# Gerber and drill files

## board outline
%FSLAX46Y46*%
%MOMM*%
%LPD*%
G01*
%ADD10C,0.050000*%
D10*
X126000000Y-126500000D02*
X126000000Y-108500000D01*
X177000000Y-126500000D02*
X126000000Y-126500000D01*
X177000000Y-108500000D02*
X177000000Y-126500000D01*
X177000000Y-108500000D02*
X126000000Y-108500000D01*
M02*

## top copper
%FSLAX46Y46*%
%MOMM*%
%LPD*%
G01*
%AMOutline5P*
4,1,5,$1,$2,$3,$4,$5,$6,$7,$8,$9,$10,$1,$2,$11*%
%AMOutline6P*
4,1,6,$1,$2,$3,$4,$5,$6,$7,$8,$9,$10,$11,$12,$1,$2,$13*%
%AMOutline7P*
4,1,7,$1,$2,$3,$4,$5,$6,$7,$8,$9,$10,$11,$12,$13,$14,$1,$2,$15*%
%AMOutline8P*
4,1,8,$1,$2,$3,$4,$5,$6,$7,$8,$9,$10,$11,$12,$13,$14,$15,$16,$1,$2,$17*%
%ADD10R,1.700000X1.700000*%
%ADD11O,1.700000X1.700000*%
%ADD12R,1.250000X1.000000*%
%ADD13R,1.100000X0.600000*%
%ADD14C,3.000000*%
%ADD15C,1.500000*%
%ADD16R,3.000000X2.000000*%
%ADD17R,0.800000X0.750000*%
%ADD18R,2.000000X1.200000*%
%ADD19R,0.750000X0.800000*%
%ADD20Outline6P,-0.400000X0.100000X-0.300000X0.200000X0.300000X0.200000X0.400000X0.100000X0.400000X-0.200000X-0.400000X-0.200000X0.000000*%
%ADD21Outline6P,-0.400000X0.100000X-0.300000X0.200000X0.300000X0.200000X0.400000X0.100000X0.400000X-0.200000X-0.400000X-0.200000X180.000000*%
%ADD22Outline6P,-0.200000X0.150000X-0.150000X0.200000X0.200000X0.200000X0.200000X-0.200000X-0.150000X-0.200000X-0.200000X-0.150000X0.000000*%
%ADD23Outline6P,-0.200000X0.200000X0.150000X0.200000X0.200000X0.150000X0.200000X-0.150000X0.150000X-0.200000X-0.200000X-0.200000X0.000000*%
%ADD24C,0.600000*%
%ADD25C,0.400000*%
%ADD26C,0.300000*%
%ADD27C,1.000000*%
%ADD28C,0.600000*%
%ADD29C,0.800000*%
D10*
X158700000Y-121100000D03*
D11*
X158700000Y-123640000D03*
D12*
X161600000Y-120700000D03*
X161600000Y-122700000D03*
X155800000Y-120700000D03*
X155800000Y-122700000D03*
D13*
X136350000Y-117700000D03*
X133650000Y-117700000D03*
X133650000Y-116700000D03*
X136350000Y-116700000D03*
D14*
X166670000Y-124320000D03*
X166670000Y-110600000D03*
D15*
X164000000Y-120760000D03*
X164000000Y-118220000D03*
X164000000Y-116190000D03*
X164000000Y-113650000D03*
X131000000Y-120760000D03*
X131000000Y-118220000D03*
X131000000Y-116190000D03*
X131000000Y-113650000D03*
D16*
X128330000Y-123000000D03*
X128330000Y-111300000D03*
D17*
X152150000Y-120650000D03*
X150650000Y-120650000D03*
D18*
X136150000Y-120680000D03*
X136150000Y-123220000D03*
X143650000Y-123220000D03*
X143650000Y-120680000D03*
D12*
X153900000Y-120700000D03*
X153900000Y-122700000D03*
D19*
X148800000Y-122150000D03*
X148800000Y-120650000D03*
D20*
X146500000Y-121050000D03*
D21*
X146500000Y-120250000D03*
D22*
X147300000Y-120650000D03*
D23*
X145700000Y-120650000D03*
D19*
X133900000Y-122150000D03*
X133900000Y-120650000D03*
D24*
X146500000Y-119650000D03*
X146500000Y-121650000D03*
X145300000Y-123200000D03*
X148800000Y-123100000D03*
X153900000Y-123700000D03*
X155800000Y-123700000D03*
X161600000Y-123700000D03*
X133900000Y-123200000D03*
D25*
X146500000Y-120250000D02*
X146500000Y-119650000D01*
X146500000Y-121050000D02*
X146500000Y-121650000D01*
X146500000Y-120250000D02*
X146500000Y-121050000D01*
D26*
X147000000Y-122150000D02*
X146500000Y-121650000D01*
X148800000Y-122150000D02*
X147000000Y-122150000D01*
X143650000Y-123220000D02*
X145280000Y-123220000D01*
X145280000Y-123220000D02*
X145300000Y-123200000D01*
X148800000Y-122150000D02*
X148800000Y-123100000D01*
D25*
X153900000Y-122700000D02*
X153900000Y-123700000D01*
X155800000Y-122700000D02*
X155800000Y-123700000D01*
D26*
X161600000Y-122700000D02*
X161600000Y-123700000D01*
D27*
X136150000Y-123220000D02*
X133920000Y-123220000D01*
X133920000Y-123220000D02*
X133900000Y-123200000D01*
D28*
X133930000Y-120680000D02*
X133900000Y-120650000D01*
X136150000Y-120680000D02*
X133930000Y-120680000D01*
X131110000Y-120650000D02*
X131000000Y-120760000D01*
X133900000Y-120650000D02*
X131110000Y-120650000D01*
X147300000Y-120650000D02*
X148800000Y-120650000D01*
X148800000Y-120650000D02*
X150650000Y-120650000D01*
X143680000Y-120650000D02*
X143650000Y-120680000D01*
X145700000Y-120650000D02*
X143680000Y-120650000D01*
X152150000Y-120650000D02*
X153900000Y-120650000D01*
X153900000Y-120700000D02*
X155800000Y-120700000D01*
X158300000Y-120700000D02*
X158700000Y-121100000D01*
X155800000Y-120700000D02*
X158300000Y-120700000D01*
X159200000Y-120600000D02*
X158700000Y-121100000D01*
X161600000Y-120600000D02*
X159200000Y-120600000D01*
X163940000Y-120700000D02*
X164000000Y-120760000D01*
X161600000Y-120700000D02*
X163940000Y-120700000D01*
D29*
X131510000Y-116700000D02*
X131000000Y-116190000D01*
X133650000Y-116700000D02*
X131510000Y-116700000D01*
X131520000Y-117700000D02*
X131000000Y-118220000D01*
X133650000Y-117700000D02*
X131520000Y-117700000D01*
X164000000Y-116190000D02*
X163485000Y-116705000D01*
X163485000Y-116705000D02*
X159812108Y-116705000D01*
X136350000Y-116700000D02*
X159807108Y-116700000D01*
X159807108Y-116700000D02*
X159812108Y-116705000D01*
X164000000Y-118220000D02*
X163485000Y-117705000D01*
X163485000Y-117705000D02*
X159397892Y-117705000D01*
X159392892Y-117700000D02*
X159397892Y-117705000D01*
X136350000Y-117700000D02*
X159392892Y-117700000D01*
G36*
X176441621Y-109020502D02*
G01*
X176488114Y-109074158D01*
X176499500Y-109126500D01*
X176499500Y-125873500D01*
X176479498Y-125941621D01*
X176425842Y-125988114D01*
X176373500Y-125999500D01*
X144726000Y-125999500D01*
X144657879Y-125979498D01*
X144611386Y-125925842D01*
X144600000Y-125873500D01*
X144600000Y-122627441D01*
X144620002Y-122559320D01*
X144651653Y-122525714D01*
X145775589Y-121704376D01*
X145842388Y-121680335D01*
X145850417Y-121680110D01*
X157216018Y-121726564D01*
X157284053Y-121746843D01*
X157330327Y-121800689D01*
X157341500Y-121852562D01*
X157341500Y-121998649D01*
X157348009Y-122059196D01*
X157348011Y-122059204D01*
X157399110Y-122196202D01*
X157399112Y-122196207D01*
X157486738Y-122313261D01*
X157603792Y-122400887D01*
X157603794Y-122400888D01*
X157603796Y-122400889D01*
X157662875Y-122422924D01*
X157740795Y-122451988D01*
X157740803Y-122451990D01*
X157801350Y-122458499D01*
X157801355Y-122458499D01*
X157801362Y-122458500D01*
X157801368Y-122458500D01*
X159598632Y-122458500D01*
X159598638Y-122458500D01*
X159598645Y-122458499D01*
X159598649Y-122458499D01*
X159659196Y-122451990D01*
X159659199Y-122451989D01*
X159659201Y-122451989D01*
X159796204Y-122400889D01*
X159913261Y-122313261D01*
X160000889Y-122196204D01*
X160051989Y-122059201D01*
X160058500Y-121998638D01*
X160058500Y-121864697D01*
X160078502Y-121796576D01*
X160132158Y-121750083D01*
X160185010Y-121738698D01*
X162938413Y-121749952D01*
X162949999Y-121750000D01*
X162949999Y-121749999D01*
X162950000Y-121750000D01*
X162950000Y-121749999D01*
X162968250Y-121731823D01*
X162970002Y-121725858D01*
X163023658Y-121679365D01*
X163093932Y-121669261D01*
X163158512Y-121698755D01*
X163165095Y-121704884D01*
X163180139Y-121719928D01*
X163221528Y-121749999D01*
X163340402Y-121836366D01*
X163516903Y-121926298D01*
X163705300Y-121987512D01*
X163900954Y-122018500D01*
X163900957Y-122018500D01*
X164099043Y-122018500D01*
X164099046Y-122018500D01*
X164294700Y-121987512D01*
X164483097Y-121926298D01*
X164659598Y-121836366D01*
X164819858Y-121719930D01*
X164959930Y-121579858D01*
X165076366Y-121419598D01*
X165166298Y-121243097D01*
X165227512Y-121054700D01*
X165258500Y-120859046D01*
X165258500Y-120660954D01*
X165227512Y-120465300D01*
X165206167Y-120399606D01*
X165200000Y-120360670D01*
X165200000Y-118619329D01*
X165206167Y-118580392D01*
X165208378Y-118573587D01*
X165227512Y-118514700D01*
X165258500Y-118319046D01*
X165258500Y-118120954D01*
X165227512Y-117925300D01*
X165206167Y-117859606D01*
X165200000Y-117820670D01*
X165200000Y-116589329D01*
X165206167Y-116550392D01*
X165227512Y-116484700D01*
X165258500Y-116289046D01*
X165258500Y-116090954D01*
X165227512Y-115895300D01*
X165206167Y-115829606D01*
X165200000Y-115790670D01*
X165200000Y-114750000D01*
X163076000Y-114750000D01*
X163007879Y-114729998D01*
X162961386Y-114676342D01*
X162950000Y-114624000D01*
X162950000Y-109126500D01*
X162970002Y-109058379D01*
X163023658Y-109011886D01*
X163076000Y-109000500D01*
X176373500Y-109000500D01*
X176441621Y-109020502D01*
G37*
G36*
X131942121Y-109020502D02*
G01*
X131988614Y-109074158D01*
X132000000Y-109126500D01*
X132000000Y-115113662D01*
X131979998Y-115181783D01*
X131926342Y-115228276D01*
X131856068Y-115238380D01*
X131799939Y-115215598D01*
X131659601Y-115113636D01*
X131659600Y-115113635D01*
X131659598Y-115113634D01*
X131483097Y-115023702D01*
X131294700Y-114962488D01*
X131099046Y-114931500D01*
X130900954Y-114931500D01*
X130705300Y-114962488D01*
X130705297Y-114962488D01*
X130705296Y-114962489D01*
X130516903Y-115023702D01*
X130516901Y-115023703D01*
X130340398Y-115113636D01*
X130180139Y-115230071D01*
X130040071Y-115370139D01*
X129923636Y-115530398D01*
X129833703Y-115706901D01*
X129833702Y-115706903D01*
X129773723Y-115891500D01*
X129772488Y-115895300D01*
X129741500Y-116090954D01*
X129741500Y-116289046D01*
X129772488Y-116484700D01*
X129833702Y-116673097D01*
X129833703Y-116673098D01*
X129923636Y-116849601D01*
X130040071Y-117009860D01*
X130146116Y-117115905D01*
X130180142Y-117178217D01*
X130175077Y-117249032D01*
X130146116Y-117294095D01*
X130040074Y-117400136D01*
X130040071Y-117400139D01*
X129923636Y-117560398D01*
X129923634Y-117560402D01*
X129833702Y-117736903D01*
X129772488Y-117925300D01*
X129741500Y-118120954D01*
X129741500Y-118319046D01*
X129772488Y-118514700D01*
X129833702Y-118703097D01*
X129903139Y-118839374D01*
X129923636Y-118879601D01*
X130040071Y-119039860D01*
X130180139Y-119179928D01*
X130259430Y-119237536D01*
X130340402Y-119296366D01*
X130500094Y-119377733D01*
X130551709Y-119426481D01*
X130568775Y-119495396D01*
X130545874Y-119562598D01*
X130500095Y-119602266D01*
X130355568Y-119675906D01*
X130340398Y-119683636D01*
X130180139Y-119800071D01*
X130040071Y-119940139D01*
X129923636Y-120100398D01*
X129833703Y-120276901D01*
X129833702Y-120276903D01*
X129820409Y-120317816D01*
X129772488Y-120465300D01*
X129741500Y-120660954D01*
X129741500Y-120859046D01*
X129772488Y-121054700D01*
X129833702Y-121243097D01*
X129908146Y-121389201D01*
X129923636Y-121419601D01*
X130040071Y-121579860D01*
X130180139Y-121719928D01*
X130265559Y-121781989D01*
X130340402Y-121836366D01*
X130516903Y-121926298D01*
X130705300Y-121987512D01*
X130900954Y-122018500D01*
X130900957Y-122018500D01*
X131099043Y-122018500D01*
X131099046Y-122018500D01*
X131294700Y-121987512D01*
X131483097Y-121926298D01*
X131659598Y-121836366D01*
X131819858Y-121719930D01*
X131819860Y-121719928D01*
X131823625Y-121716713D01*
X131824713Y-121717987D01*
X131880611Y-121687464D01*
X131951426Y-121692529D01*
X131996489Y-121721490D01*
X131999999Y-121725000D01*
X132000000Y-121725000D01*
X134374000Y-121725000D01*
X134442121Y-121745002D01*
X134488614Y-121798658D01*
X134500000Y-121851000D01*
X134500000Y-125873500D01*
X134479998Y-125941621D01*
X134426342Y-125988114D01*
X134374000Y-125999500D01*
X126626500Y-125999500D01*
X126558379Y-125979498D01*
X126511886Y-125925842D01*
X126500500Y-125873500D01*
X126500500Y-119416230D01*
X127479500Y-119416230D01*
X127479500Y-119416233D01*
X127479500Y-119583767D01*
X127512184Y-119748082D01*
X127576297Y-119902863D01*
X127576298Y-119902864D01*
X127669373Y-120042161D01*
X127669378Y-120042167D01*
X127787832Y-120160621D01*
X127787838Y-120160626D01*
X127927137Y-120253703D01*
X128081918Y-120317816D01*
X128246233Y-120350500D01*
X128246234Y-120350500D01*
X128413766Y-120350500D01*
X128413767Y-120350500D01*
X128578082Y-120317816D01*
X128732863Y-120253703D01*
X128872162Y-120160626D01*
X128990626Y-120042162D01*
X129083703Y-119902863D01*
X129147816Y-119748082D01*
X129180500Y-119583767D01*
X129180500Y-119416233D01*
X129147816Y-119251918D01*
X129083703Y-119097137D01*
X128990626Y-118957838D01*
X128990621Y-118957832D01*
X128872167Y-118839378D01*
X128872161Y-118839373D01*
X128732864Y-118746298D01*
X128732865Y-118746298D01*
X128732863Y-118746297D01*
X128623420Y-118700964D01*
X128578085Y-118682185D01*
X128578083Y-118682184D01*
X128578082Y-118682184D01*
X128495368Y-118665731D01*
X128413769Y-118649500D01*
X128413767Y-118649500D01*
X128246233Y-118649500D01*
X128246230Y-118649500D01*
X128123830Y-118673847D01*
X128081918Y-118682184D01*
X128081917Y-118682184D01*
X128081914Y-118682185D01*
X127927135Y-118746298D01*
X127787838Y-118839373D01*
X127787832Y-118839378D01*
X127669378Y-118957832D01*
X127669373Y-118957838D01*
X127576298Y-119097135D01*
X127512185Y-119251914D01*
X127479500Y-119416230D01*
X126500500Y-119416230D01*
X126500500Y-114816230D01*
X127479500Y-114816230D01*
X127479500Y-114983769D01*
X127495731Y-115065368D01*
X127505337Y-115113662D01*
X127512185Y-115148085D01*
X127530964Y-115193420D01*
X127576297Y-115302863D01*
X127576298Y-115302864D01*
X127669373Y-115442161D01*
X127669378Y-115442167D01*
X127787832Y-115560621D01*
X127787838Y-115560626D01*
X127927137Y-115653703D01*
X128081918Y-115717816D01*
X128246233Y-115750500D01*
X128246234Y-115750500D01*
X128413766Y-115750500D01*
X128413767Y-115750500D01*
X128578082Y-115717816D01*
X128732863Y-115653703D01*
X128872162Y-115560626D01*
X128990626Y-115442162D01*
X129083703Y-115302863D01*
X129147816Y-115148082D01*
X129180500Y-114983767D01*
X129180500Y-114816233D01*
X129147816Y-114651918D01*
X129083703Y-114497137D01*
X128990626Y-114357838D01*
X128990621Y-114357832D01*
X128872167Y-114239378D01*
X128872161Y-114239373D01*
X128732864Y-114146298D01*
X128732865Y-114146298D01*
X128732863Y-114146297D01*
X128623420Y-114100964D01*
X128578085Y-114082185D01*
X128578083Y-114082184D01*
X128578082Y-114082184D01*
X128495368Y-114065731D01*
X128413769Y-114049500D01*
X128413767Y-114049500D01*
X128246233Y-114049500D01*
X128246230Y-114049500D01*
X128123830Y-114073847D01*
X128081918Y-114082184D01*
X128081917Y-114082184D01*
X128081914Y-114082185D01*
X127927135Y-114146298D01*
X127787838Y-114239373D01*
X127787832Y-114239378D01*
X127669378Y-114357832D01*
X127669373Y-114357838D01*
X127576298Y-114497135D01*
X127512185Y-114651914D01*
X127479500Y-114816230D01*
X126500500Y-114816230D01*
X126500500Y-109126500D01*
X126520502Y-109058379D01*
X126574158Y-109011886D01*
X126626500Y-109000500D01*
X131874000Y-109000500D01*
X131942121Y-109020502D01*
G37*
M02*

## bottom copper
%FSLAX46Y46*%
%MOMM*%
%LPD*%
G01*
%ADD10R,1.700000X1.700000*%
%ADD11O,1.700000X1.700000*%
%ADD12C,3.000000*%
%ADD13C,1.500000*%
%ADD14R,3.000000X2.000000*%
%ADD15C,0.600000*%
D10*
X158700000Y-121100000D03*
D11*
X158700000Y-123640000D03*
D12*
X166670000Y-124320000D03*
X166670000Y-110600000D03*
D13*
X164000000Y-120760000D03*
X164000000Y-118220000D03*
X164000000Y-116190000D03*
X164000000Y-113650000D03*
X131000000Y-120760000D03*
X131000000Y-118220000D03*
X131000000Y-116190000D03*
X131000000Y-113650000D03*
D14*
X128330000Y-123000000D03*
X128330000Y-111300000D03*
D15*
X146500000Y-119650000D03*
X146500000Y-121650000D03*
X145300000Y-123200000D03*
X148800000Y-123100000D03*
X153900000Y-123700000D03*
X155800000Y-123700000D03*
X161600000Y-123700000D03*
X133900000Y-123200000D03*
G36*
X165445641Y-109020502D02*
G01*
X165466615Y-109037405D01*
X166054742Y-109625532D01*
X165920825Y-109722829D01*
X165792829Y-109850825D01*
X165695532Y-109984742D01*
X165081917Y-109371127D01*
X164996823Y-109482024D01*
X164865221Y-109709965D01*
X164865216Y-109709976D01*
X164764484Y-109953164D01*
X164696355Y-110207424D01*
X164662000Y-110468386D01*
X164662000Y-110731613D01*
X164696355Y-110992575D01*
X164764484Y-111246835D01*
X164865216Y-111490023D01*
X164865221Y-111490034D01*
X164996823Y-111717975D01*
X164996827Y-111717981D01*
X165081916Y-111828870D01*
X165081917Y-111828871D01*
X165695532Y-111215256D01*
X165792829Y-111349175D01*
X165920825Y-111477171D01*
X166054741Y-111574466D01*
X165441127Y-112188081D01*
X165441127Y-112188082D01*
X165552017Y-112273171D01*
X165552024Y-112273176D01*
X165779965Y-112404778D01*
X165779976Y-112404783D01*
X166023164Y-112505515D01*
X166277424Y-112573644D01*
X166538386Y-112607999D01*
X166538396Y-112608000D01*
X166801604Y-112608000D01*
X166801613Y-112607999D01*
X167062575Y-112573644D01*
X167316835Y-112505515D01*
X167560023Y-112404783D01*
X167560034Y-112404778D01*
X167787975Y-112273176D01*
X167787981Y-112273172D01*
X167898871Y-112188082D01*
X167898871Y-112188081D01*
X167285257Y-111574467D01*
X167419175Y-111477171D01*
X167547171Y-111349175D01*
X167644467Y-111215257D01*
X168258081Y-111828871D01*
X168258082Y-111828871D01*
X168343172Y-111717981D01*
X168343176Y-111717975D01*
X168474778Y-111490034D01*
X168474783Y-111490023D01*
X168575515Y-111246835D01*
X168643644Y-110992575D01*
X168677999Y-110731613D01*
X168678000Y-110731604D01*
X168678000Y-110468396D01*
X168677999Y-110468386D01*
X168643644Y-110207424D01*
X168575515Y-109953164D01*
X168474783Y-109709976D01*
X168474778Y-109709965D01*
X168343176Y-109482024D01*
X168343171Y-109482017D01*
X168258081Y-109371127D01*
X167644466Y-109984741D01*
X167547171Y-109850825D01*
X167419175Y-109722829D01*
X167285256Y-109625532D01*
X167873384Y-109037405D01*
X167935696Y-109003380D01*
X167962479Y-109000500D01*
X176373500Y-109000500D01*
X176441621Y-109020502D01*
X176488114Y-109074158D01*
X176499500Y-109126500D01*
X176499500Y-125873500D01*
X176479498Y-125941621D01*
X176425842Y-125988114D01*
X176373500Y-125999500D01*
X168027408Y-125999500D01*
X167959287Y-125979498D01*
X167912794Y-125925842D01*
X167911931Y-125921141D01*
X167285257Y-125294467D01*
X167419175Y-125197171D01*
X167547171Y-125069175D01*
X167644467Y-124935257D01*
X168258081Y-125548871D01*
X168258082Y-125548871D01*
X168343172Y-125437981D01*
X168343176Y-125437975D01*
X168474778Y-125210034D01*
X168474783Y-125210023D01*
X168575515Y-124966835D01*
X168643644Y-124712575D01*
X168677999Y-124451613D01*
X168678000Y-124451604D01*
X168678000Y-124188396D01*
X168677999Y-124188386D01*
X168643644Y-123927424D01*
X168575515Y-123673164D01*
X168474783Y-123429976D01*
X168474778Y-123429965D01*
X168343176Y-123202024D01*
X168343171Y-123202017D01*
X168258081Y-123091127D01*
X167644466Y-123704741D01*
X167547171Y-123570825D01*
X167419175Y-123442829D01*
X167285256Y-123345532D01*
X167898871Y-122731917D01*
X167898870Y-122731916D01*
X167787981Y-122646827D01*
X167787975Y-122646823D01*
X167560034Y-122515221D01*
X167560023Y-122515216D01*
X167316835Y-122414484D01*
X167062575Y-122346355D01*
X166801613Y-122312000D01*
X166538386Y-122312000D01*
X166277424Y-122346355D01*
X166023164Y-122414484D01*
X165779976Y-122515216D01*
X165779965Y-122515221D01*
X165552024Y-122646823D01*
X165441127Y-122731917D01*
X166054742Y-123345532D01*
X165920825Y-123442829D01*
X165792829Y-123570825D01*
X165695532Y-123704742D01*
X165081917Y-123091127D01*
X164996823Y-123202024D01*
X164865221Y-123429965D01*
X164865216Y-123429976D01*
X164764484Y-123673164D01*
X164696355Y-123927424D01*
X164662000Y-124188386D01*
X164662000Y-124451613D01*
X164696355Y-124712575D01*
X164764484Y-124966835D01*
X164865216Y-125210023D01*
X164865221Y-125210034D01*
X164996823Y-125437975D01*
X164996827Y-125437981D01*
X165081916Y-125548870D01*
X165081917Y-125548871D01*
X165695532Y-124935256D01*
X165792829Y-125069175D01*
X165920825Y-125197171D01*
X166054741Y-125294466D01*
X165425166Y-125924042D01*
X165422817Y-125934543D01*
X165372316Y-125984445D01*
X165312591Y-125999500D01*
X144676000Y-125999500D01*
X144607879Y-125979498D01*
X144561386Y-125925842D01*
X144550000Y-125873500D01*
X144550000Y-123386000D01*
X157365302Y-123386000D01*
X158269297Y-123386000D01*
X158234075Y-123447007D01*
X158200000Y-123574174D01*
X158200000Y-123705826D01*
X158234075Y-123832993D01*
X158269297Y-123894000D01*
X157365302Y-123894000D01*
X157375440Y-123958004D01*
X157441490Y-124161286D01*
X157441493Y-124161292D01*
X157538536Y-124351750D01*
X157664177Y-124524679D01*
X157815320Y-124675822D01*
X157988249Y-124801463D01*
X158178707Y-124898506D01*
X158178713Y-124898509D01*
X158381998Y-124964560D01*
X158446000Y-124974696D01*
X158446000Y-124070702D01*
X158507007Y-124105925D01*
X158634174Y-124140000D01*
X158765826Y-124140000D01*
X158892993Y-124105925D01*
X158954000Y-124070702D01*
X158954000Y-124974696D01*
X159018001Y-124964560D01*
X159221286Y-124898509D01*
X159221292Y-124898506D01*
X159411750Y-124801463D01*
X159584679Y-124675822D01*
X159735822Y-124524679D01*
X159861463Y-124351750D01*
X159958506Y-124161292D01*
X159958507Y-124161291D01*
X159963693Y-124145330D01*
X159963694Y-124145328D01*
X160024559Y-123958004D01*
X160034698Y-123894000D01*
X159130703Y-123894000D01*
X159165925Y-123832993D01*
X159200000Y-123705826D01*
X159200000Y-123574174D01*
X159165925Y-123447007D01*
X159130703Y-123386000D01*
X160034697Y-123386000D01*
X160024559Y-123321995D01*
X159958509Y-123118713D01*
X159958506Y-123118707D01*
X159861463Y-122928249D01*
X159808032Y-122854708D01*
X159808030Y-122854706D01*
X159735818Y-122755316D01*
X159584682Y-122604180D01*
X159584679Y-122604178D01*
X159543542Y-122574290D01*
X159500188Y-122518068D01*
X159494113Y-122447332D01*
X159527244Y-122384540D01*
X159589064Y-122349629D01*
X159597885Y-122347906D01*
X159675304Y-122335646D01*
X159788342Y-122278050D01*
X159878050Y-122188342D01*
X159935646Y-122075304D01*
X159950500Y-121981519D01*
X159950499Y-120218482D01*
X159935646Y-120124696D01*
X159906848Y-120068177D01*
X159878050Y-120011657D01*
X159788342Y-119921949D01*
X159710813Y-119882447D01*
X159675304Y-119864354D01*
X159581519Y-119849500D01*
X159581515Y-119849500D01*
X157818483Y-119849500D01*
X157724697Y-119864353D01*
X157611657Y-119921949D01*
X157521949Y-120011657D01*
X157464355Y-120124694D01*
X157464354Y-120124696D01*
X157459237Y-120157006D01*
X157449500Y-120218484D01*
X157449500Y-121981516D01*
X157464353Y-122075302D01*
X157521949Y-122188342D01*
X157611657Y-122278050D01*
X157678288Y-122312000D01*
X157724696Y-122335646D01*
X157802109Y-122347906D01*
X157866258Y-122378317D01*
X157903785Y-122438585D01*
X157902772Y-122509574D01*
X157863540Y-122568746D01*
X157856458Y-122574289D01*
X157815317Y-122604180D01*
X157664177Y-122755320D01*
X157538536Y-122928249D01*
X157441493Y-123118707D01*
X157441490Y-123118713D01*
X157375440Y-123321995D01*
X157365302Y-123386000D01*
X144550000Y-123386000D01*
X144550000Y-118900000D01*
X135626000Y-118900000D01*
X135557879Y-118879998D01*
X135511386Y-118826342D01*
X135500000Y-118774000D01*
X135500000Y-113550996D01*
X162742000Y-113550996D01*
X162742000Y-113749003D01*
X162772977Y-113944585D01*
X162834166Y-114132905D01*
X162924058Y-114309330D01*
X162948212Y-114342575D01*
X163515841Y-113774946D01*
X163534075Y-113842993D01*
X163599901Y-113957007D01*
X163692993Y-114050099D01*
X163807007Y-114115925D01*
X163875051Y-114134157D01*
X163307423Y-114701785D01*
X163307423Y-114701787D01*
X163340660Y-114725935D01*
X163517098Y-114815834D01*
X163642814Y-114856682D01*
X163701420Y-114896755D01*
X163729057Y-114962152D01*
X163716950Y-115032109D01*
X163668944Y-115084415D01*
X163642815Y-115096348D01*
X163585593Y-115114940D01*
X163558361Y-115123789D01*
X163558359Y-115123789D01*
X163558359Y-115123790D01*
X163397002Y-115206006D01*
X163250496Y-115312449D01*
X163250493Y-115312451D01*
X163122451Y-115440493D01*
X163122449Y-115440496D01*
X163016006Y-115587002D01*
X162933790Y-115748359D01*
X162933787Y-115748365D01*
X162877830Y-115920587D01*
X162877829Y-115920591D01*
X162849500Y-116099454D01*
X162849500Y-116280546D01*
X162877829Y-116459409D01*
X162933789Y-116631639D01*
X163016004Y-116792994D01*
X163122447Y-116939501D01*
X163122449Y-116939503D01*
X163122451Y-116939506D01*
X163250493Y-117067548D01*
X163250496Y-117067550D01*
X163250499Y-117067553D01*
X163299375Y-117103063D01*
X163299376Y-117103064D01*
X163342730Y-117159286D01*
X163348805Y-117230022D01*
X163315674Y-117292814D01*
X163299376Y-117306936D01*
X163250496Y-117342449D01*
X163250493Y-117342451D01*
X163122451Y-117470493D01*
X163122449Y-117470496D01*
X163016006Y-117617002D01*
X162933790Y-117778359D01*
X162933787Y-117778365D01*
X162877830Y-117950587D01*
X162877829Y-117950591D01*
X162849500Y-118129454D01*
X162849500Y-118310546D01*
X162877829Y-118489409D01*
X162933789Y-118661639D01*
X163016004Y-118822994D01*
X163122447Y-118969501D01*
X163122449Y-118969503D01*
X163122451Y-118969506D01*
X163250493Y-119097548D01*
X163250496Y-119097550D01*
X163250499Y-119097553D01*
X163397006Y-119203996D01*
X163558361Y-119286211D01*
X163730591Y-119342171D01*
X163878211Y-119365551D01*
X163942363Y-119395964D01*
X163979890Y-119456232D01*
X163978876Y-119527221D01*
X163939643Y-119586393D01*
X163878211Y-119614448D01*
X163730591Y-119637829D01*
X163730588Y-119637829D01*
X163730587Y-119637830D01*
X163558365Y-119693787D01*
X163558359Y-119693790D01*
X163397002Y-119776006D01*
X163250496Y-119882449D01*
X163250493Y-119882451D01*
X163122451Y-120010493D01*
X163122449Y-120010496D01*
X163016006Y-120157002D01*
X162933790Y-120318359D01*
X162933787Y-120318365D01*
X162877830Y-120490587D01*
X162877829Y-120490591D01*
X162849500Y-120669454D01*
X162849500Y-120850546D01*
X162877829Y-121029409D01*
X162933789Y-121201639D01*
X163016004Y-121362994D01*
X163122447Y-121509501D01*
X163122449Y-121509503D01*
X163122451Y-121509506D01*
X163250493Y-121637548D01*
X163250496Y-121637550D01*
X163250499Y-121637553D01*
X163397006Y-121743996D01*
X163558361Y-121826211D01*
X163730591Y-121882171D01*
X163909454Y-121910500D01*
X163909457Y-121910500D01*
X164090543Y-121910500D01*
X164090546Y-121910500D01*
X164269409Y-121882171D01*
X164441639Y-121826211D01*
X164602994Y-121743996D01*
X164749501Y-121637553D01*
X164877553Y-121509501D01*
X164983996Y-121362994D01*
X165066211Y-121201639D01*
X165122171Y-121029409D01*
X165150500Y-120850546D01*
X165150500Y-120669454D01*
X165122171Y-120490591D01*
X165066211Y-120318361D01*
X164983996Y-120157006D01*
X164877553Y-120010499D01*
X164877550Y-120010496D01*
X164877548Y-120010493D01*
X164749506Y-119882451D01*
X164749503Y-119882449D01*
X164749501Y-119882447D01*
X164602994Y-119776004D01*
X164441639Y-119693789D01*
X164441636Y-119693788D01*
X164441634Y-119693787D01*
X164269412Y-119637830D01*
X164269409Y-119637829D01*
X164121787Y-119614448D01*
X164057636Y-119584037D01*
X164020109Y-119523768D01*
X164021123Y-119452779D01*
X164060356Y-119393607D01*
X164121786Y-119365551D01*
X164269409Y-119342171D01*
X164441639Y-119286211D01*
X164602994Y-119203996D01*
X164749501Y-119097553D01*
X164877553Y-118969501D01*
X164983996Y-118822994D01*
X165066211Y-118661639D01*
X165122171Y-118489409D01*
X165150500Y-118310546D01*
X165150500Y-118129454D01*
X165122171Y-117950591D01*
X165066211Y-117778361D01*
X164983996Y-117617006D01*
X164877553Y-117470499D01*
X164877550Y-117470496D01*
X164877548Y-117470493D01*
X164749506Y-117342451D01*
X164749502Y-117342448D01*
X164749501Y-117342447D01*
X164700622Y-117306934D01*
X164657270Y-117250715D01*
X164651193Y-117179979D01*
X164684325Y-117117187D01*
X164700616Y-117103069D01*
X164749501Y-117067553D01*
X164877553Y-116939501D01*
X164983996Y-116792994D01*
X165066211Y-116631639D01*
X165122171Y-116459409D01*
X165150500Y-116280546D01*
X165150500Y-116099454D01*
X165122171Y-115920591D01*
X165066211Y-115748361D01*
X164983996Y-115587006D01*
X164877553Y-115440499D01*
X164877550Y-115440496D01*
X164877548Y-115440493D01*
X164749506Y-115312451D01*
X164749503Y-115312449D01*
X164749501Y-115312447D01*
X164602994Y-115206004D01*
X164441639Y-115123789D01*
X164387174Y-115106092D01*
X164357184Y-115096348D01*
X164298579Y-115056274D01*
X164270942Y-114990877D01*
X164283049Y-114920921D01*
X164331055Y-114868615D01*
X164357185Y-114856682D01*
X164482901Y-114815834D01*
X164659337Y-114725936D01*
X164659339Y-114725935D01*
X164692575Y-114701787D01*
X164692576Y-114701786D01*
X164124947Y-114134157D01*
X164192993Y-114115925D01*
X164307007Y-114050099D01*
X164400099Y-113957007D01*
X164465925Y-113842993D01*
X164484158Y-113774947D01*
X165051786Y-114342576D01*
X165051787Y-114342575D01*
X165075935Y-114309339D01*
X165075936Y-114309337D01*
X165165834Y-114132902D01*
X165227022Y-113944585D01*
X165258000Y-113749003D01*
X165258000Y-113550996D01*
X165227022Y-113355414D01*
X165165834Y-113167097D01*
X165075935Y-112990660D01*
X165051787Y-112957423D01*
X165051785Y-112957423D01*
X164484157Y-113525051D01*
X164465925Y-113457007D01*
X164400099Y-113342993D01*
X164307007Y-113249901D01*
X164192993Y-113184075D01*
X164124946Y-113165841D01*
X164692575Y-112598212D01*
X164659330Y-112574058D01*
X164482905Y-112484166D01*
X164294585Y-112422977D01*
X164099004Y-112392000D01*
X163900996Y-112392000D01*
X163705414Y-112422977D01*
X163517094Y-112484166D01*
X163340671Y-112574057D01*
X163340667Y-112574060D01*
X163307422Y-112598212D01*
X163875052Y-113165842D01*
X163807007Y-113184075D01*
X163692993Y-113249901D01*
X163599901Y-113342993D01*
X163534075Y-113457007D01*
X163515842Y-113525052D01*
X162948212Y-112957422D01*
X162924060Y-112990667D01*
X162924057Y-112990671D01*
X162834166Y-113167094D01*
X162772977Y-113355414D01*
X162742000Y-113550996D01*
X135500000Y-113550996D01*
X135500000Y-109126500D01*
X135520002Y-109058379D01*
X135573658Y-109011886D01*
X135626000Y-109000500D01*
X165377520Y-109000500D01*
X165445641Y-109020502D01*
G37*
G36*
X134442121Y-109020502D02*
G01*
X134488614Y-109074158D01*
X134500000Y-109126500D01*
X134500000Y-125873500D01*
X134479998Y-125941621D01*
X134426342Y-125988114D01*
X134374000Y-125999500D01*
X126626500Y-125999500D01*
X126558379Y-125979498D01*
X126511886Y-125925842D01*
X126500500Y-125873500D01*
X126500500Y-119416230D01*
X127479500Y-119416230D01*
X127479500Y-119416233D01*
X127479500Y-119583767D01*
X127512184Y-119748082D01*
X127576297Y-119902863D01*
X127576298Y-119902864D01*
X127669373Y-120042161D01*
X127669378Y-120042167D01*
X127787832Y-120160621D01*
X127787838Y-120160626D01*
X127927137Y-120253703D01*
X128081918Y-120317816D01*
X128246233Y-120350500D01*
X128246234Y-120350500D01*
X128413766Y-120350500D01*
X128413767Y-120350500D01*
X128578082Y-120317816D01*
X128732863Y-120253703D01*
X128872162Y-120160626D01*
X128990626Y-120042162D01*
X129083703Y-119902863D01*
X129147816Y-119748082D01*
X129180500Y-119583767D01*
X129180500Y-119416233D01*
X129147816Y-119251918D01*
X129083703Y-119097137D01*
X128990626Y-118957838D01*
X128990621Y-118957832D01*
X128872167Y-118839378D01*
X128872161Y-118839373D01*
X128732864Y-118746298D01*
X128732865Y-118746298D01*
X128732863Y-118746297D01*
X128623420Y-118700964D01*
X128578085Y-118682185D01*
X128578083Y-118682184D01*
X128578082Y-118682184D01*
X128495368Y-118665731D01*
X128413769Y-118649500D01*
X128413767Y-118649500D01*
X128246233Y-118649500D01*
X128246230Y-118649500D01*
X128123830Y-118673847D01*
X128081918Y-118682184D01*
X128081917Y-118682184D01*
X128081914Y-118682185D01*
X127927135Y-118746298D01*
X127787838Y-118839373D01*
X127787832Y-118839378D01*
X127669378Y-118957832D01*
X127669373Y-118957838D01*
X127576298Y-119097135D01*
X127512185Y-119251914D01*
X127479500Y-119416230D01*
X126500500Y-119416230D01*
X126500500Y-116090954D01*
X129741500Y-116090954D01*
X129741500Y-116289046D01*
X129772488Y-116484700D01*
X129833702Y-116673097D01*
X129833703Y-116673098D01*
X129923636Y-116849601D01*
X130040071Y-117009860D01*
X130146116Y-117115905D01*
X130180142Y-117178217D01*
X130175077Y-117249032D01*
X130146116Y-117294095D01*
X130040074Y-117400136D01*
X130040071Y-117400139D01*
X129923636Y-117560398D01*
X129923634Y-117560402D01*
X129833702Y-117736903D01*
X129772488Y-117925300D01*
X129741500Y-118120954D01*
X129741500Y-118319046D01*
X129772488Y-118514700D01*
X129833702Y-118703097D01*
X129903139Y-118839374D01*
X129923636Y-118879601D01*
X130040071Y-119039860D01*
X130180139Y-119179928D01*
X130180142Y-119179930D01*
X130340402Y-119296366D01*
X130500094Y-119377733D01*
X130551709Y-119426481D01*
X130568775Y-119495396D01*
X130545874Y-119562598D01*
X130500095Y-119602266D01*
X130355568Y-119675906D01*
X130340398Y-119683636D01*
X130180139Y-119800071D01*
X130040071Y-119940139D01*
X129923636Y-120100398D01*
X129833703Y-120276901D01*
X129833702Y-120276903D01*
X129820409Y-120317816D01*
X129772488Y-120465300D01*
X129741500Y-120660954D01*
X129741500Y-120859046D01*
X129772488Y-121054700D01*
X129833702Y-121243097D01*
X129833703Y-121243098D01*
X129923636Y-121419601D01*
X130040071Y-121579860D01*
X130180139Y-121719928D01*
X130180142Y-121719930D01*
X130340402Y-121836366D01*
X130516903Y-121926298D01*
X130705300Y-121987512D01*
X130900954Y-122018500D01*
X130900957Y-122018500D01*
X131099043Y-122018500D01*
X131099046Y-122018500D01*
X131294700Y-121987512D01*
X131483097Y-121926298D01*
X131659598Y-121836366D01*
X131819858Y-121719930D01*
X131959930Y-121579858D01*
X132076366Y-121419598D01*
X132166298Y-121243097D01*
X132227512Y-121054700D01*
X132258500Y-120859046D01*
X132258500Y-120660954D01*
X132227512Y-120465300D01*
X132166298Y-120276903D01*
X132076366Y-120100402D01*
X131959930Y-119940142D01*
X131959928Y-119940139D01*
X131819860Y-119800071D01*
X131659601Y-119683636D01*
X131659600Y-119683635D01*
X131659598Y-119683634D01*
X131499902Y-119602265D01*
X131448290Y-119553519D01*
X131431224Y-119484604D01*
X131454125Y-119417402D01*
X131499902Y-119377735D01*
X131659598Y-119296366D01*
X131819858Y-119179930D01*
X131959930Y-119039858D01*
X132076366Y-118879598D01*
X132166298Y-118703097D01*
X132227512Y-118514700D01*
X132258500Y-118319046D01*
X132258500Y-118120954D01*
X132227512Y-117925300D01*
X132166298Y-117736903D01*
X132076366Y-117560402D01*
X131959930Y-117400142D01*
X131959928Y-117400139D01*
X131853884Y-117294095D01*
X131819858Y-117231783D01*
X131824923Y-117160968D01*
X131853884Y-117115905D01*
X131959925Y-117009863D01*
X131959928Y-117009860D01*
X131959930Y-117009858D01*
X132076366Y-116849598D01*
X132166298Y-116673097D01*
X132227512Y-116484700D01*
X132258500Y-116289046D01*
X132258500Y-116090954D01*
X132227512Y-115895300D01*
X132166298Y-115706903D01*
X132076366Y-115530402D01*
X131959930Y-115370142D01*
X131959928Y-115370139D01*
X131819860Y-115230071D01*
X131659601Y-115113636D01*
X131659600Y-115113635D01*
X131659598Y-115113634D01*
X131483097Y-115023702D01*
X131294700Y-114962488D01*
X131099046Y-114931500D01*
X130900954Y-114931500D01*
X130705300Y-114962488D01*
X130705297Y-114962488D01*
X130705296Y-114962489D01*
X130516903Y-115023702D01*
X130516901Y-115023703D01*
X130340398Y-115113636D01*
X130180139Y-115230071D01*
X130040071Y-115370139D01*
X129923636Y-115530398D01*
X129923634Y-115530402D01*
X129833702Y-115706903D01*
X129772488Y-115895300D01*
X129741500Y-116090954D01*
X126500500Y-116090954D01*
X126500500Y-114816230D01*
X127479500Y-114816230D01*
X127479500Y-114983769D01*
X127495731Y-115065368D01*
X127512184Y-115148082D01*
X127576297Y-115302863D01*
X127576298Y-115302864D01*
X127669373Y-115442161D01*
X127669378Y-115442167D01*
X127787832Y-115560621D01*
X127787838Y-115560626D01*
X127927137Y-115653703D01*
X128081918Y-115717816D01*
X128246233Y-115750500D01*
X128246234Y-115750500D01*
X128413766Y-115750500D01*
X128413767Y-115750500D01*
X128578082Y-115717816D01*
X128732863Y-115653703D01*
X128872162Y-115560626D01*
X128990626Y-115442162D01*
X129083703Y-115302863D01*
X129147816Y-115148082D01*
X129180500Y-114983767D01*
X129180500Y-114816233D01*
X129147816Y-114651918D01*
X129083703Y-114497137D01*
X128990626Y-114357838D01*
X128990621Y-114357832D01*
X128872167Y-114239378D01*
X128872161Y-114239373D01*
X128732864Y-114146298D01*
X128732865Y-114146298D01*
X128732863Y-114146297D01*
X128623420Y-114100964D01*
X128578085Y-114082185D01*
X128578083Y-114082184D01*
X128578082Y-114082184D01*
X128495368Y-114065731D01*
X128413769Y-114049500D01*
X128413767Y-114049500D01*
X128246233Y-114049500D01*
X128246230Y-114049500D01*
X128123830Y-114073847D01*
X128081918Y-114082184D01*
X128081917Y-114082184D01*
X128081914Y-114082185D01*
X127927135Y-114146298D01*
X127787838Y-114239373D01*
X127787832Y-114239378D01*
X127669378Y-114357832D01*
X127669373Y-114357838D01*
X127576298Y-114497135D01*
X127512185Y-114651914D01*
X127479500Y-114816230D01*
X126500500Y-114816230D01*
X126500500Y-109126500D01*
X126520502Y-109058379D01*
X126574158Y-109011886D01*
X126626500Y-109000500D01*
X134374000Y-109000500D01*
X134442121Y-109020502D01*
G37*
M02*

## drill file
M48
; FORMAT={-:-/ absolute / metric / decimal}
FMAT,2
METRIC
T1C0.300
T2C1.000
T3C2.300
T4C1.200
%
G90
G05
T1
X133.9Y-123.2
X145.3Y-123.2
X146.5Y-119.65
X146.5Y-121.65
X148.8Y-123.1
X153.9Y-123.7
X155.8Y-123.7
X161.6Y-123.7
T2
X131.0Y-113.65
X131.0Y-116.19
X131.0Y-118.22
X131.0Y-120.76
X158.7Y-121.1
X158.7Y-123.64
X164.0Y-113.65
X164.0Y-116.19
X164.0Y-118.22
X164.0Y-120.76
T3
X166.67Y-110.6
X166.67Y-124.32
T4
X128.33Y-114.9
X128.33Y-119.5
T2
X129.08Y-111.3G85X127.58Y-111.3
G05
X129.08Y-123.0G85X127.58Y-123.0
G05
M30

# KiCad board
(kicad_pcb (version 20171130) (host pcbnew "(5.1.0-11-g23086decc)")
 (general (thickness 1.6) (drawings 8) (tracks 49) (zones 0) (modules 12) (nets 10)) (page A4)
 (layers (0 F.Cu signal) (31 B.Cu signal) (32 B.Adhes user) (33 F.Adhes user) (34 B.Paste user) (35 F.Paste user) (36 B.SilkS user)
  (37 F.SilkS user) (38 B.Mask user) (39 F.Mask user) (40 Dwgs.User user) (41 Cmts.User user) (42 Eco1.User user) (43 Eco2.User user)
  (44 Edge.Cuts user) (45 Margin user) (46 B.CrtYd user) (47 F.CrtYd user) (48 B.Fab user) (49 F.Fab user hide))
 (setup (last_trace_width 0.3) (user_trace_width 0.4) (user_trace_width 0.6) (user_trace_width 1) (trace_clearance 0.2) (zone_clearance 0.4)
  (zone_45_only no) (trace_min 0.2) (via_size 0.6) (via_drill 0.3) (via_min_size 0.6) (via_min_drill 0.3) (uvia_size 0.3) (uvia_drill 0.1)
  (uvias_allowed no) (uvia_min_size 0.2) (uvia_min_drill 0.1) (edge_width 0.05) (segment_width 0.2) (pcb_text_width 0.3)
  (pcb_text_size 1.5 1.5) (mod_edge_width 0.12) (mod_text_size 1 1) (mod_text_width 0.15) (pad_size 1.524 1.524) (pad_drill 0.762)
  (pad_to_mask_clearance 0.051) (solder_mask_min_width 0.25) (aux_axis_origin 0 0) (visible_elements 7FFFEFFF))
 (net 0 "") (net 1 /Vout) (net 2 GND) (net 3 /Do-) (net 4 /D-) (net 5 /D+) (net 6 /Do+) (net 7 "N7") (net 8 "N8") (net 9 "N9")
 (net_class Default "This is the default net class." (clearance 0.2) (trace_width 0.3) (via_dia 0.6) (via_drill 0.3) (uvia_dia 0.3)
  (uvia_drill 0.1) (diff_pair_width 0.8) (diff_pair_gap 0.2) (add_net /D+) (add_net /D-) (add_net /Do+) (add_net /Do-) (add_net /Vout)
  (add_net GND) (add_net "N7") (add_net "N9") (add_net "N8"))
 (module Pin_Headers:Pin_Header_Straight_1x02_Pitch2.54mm (layer F.Cu) (at 158.7 121.1)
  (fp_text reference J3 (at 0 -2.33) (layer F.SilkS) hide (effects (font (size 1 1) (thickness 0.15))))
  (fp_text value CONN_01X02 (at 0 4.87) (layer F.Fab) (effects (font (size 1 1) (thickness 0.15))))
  (pad 1 thru_hole rect (at 0 0) (size 1.7 1.7) (drill 1) (layers *.Cu *.Mask) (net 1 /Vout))
  (pad 2 thru_hole oval (at 0 2.54) (size 1.7 1.7) (drill 1) (layers *.Cu *.Mask) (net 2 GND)))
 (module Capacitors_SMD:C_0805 (layer F.Cu) (at 161.6 121.7 270)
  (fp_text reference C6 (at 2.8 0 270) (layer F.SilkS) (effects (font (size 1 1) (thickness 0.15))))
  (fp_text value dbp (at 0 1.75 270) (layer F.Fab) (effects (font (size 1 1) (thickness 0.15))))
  (pad 1 smd rect (at -1 0 270) (size 1 1.25) (layers F.Cu F.Paste F.Mask) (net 1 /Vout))
  (pad 2 smd rect (at 1 0 270) (size 1 1.25) (layers F.Cu F.Paste F.Mask) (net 2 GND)))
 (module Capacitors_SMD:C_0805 (layer F.Cu) (at 155.8 121.7 270)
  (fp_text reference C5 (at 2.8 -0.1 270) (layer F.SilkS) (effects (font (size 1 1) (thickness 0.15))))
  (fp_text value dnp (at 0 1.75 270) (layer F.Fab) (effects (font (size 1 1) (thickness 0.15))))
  (pad 1 smd rect (at -1 0 270) (size 1 1.25) (layers F.Cu F.Paste F.Mask) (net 1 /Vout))
  (pad 2 smd rect (at 1 0 270) (size 1 1.25) (layers F.Cu F.Paste F.Mask) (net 2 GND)))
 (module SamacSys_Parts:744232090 (layer F.Cu) (at 135 117.2 180)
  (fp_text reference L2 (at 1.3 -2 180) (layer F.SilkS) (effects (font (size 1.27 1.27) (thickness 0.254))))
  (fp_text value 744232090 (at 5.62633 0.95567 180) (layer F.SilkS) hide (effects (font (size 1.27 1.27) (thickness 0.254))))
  (pad 4 smd rect (at -1.35 -0.5 270) (size 0.6 1.1) (layers F.Cu F.Paste) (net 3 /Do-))
  (pad 3 smd rect (at 1.35 -0.5 270) (size 0.6 1.1) (layers F.Cu F.Paste) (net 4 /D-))
  (pad 2 smd rect (at 1.35 0.5 270) (size 0.6 1.1) (layers F.Cu F.Paste) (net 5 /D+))
  (pad 1 smd rect (at -1.35 0.5 270) (size 0.6 1.1) (layers F.Cu F.Paste) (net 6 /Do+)))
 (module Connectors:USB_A (layer F.Cu) (at 164 120.76 90)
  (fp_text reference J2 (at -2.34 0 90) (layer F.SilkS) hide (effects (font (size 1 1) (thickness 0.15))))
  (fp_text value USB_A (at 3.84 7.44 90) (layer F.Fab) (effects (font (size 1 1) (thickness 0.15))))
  (pad 5 thru_hole circle (at -3.56 2.67) (size 3 3) (drill 2.3) (layers *.Cu *.Mask) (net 2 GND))
  (pad 5 thru_hole circle (at 10.16 2.67) (size 3 3) (drill 2.3) (layers *.Cu *.Mask) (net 2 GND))
  (pad 1 thru_hole circle (at 0 0) (size 1.5 1.5) (drill 1) (layers *.Cu *.Mask) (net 1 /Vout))
  (pad 2 thru_hole circle (at 2.54 0) (size 1.5 1.5) (drill 1) (layers *.Cu *.Mask) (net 3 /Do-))
  (pad 3 thru_hole circle (at 4.57 0) (size 1.5 1.5) (drill 1) (layers *.Cu *.Mask) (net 6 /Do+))
  (pad 4 thru_hole circle (at 7.11 0) (size 1.5 1.5) (drill 1) (layers *.Cu *.Mask) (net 2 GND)))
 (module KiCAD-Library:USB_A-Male (layer F.Cu) (at 131 113.65 270)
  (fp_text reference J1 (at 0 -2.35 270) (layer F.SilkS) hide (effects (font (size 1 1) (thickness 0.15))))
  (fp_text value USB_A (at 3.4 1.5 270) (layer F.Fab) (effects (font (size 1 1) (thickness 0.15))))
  (pad "" np_thru_hole circle (at 5.85 2.67 180) (size 1.2 1.2) (drill 1.2) (layers *.Cu *.Mask))
  (pad "" np_thru_hole circle (at 1.25 2.67 180) (size 1.2 1.2) (drill 1.2) (layers *.Cu *.Mask))
  (pad 1 thru_hole circle (at 7.11 0 180) (size 1.5 1.5) (drill 1) (layers *.Cu *.Mask) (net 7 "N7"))
  (pad 2 thru_hole circle (at 4.57 0 180) (size 1.5 1.5) (drill 1) (layers *.Cu *.Mask) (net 4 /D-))
  (pad 3 thru_hole circle (at 2.54 0 180) (size 1.5 1.5) (drill 1) (layers *.Cu *.Mask) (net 5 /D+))
  (pad 4 thru_hole circle (at 0 0 180) (size 1.5 1.5) (drill 1) (layers *.Cu *.Mask) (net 2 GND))
  (pad 5 thru_hole rect (at 9.35 2.67 180) (size 3 2) (drill oval 2.5 1) (layers *.Cu *.Mask) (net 2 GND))
  (pad 5 thru_hole rect (at -2.35 2.67 180) (size 3 2) (drill oval 2.5 1) (layers *.Cu *.Mask) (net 2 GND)))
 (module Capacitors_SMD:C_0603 (layer F.Cu) (at 151.4 120.65)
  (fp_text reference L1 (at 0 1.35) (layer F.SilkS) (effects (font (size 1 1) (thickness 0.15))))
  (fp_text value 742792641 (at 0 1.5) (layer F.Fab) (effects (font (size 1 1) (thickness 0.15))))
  (pad 2 smd rect (at 0.75 0) (size 0.8 0.75) (layers F.Cu F.Paste F.Mask) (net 1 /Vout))
  (pad 1 smd rect (at -0.75 0) (size 0.8 0.75) (layers F.Cu F.Paste F.Mask) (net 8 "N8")))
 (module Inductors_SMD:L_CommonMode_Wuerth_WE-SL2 (layer F.Cu) (at 139.9 121.95)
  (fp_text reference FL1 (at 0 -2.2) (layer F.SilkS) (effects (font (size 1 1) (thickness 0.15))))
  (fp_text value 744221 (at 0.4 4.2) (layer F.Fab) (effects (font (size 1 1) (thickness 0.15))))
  (pad 1 smd rect (at -3.75 -1.27) (size 2 1.2) (layers F.Cu F.Paste F.Mask) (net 7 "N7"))
  (pad 2 smd rect (at -3.75 1.27) (size 2 1.2) (layers F.Cu F.Paste F.Mask) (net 2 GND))
  (pad 3 smd rect (at 3.75 1.27) (size 2 1.2) (layers F.Cu F.Paste F.Mask) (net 2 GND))
  (pad 4 smd rect (at 3.75 -1.27) (size 2 1.2) (layers F.Cu F.Paste F.Mask) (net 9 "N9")))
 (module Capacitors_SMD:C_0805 (layer F.Cu) (at 153.9 121.7 270)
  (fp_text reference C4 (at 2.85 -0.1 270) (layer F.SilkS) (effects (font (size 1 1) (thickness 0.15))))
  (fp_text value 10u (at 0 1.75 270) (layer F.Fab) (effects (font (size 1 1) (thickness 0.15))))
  (pad 1 smd rect (at -1 0 270) (size 1 1.25) (layers F.Cu F.Paste F.Mask) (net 1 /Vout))
  (pad 2 smd rect (at 1 0 270) (size 1 1.25) (layers F.Cu F.Paste F.Mask) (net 2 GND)))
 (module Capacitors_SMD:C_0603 (layer F.Cu) (at 148.8 121.4 270)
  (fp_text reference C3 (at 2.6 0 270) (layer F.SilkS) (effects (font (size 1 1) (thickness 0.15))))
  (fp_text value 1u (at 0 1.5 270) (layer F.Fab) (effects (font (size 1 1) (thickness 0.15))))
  (pad 2 smd rect (at 0.75 0 270) (size 0.8 0.75) (layers F.Cu F.Paste F.Mask) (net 2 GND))
  (pad 1 smd rect (at -0.75 0 270) (size 0.8 0.75) (layers F.Cu F.Paste F.Mask) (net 8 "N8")))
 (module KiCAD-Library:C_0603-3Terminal (layer F.Cu) (at 146.5 120.65)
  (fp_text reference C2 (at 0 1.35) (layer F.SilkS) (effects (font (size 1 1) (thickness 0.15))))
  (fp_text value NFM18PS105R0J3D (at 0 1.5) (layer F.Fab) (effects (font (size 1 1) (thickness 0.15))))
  (pad 2 smd roundrect (at 0 0.4) (size 0.8 0.4) (layers F.Cu F.Paste F.Mask) (roundrect_rratio 0) (chamfer_ratio 0.25)
   (chamfer top_left top_right) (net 2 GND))
  (pad 2 smd roundrect (at 0 -0.4 180) (size 0.8 0.4) (layers F.Cu F.Paste F.Mask) (roundrect_rratio 0) (chamfer_ratio 0.25)
   (chamfer top_left top_right) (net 2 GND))
  (pad 3 smd roundrect (at 0.8 0) (size 0.4 0.4) (layers F.Cu F.Paste F.Mask) (roundrect_rratio 0) (chamfer_ratio 0.125)
   (chamfer top_left bottom_left) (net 8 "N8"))
  (pad 1 smd roundrect (at -0.8 0) (size 0.4 0.4) (layers F.Cu F.Paste F.Mask) (roundrect_rratio 0) (chamfer_ratio 0.125)
   (chamfer top_right bottom_right) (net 9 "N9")))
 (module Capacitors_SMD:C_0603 (layer F.Cu) (at 133.9 121.4 270)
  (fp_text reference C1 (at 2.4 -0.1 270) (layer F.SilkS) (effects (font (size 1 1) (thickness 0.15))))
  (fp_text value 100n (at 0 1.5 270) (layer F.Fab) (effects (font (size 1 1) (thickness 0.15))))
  (pad 2 smd rect (at 0.75 0 270) (size 0.8 0.75) (layers F.Cu F.Paste F.Mask) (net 2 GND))
  (pad 1 smd rect (at -0.75 0 270) (size 0.8 0.75) (layers F.Cu F.Paste F.Mask) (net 7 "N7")))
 (gr_line (start 126 126.5) (end 126 108.5) (layer Edge.Cuts) (width 0.05))
 (gr_line (start 177 126.5) (end 126 126.5) (layer Edge.Cuts) (width 0.05))
 (gr_line (start 177 108.5) (end 177 126.5) (layer Edge.Cuts) (width 0.05))
 (gr_line (start 177 108.5) (end 126 108.5) (layer Edge.Cuts) (width 0.05))
 (via (at 146.5 119.65) (size 0.6) (drill 0.3) (layers F.Cu B.Cu) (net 2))
 (segment (start 146.5 120.25) (end 146.5 119.65) (width 0.4) (layer F.Cu) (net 2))
 (via (at 146.5 121.65) (size 0.6) (drill 0.3) (layers F.Cu B.Cu) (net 2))
 (segment (start 146.5 121.05) (end 146.5 121.65) (width 0.4) (layer F.Cu) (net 2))
 (segment (start 146.5 120.25) (end 146.5 121.05) (width 0.4) (layer F.Cu) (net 2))
 (segment (start 147 122.15) (end 146.5 121.65) (width 0.3) (layer F.Cu) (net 2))
 (segment (start 148.8 122.15) (end 147 122.15) (width 0.3) (layer F.Cu) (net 2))
 (via (at 145.3 123.2) (size 0.6) (drill 0.3) (layers F.Cu B.Cu) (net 2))
 (segment (start 143.65 123.22) (end 145.28 123.22) (width 0.3) (layer F.Cu) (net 2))
 (segment (start 145.28 123.22) (end 145.3 123.2) (width 0.3) (layer F.Cu) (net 2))
 (via (at 148.8 123.1) (size 0.6) (drill 0.3) (layers F.Cu B.Cu) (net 2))
 (segment (start 148.8 122.15) (end 148.8 123.1) (width 0.3) (layer F.Cu) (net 2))
 (via (at 153.9 123.7) (size 0.6) (drill 0.3) (layers F.Cu B.Cu) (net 2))
 (segment (start 153.9 122.7) (end 153.9 123.7) (width 0.4) (layer F.Cu) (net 2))
 (via (at 155.8 123.7) (size 0.6) (drill 0.3) (layers F.Cu B.Cu) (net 2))
 (segment (start 155.8 122.7) (end 155.8 123.7) (width 0.4) (layer F.Cu) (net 2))
 (via (at 161.6 123.7) (size 0.6) (drill 0.3) (layers F.Cu B.Cu) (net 2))
 (segment (start 161.6 122.7) (end 161.6 123.7) (width 0.3) (layer F.Cu) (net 2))
 (via (at 133.9 123.2) (size 0.6) (drill 0.3) (layers F.Cu B.Cu) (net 2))
 (segment (start 136.15 123.22) (end 133.92 123.22) (width 1) (layer F.Cu) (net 2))
 (segment (start 133.92 123.22) (end 133.9 123.2) (width 1) (layer F.Cu) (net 2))
 (segment (start 133.93 120.68) (end 133.9 120.65) (width 0.6) (layer F.Cu) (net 7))
 (segment (start 136.15 120.68) (end 133.93 120.68) (width 0.6) (layer F.Cu) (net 7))
 (segment (start 131.11 120.65) (end 131 120.76) (width 0.6) (layer F.Cu) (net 7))
 (segment (start 133.9 120.65) (end 131.11 120.65) (width 0.6) (layer F.Cu) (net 7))
 (segment (start 147.3 120.65) (end 148.8 120.65) (width 0.6) (layer F.Cu) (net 8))
 (segment (start 148.8 120.65) (end 150.65 120.65) (width 0.6) (layer F.Cu) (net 8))
 (segment (start 143.68 120.65) (end 143.65 120.68) (width 0.6) (layer F.Cu) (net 9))
 (segment (start 145.7 120.65) (end 143.68 120.65) (width 0.6) (layer F.Cu) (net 9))
 (segment (start 152.15 120.65) (end 153.9 120.65) (width 0.6) (layer F.Cu) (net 1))
 (segment (start 153.9 120.7) (end 155.8 120.7) (width 0.6) (layer F.Cu) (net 1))
 (segment (start 158.3 120.7) (end 158.7 121.1) (width 0.6) (layer F.Cu) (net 1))
 (segment (start 155.8 120.7) (end 158.3 120.7) (width 0.6) (layer F.Cu) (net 1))
 (segment (start 159.2 120.6) (end 158.7 121.1) (width 0.6) (layer F.Cu) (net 1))
 (segment (start 161.6 120.6) (end 159.2 120.6) (width 0.6) (layer F.Cu) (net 1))
 (segment (start 163.94 120.7) (end 164 120.76) (width 0.6) (layer F.Cu) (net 1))
 (segment (start 161.6 120.7) (end 163.94 120.7) (width 0.6) (layer F.Cu) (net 1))
 (segment (start 131.51 116.7) (end 131 116.19) (width 0.8) (layer F.Cu) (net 5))
 (segment (start 133.65 116.7) (end 131.51 116.7) (width 0.8) (layer F.Cu) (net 5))
 (segment (start 131.52 117.7) (end 131 118.22) (width 0.8) (layer F.Cu) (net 4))
 (segment (start 133.65 117.7) (end 131.52 117.7) (width 0.8) (layer F.Cu) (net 4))
 (segment (start 164 116.19) (end 163.485 116.705) (width 0.8) (layer F.Cu) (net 6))
 (segment (start 163.485 116.705) (end 159.812108 116.705) (width 0.8) (layer F.Cu) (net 6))
 (segment (start 136.35 116.7) (end 159.807108 116.7) (width 0.8) (layer F.Cu) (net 6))
 (segment (start 159.807108 116.7) (end 159.812108 116.705) (width 0.8) (layer F.Cu) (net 6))
 (segment (start 164 118.22) (end 163.485 117.705) (width 0.8) (layer F.Cu) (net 3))
 (segment (start 163.485 117.705) (end 159.397892 117.705) (width 0.8) (layer F.Cu) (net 3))
 (segment (start 159.392892 117.7) (end 159.397892 117.705) (width 0.8) (layer F.Cu) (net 3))
 (segment (start 136.35 117.7) (end 159.392892 117.7) (width 0.8) (layer F.Cu) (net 3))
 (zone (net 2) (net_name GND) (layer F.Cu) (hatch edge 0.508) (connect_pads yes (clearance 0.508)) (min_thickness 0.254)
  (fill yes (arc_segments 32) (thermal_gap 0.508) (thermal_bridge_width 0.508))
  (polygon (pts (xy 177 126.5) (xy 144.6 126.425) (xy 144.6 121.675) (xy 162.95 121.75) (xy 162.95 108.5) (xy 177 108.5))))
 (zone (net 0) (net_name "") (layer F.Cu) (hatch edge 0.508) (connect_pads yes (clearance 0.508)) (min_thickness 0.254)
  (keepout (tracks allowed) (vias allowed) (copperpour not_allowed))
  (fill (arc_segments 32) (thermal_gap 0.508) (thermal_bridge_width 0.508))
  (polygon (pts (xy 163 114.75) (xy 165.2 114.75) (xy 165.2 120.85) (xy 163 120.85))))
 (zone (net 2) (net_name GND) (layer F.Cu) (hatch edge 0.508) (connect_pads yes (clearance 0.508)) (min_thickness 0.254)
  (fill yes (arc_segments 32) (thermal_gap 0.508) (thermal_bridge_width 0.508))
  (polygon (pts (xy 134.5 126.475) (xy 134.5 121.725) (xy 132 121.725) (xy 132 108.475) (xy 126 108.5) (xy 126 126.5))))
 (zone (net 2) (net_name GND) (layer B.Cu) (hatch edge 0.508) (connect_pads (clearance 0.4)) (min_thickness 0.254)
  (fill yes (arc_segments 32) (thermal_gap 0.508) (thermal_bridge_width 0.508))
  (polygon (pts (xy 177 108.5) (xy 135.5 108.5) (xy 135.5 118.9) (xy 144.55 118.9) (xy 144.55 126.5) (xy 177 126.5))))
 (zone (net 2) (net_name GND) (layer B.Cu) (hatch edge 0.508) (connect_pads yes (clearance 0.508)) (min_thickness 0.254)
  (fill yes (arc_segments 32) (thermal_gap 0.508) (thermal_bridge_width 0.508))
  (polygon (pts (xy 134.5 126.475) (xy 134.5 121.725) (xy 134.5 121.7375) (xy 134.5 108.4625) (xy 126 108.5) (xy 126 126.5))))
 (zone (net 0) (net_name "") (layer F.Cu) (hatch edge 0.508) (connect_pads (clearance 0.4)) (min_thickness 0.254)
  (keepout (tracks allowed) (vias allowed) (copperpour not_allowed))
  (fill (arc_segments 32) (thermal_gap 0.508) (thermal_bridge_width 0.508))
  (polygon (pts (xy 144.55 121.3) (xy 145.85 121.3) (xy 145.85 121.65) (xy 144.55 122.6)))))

